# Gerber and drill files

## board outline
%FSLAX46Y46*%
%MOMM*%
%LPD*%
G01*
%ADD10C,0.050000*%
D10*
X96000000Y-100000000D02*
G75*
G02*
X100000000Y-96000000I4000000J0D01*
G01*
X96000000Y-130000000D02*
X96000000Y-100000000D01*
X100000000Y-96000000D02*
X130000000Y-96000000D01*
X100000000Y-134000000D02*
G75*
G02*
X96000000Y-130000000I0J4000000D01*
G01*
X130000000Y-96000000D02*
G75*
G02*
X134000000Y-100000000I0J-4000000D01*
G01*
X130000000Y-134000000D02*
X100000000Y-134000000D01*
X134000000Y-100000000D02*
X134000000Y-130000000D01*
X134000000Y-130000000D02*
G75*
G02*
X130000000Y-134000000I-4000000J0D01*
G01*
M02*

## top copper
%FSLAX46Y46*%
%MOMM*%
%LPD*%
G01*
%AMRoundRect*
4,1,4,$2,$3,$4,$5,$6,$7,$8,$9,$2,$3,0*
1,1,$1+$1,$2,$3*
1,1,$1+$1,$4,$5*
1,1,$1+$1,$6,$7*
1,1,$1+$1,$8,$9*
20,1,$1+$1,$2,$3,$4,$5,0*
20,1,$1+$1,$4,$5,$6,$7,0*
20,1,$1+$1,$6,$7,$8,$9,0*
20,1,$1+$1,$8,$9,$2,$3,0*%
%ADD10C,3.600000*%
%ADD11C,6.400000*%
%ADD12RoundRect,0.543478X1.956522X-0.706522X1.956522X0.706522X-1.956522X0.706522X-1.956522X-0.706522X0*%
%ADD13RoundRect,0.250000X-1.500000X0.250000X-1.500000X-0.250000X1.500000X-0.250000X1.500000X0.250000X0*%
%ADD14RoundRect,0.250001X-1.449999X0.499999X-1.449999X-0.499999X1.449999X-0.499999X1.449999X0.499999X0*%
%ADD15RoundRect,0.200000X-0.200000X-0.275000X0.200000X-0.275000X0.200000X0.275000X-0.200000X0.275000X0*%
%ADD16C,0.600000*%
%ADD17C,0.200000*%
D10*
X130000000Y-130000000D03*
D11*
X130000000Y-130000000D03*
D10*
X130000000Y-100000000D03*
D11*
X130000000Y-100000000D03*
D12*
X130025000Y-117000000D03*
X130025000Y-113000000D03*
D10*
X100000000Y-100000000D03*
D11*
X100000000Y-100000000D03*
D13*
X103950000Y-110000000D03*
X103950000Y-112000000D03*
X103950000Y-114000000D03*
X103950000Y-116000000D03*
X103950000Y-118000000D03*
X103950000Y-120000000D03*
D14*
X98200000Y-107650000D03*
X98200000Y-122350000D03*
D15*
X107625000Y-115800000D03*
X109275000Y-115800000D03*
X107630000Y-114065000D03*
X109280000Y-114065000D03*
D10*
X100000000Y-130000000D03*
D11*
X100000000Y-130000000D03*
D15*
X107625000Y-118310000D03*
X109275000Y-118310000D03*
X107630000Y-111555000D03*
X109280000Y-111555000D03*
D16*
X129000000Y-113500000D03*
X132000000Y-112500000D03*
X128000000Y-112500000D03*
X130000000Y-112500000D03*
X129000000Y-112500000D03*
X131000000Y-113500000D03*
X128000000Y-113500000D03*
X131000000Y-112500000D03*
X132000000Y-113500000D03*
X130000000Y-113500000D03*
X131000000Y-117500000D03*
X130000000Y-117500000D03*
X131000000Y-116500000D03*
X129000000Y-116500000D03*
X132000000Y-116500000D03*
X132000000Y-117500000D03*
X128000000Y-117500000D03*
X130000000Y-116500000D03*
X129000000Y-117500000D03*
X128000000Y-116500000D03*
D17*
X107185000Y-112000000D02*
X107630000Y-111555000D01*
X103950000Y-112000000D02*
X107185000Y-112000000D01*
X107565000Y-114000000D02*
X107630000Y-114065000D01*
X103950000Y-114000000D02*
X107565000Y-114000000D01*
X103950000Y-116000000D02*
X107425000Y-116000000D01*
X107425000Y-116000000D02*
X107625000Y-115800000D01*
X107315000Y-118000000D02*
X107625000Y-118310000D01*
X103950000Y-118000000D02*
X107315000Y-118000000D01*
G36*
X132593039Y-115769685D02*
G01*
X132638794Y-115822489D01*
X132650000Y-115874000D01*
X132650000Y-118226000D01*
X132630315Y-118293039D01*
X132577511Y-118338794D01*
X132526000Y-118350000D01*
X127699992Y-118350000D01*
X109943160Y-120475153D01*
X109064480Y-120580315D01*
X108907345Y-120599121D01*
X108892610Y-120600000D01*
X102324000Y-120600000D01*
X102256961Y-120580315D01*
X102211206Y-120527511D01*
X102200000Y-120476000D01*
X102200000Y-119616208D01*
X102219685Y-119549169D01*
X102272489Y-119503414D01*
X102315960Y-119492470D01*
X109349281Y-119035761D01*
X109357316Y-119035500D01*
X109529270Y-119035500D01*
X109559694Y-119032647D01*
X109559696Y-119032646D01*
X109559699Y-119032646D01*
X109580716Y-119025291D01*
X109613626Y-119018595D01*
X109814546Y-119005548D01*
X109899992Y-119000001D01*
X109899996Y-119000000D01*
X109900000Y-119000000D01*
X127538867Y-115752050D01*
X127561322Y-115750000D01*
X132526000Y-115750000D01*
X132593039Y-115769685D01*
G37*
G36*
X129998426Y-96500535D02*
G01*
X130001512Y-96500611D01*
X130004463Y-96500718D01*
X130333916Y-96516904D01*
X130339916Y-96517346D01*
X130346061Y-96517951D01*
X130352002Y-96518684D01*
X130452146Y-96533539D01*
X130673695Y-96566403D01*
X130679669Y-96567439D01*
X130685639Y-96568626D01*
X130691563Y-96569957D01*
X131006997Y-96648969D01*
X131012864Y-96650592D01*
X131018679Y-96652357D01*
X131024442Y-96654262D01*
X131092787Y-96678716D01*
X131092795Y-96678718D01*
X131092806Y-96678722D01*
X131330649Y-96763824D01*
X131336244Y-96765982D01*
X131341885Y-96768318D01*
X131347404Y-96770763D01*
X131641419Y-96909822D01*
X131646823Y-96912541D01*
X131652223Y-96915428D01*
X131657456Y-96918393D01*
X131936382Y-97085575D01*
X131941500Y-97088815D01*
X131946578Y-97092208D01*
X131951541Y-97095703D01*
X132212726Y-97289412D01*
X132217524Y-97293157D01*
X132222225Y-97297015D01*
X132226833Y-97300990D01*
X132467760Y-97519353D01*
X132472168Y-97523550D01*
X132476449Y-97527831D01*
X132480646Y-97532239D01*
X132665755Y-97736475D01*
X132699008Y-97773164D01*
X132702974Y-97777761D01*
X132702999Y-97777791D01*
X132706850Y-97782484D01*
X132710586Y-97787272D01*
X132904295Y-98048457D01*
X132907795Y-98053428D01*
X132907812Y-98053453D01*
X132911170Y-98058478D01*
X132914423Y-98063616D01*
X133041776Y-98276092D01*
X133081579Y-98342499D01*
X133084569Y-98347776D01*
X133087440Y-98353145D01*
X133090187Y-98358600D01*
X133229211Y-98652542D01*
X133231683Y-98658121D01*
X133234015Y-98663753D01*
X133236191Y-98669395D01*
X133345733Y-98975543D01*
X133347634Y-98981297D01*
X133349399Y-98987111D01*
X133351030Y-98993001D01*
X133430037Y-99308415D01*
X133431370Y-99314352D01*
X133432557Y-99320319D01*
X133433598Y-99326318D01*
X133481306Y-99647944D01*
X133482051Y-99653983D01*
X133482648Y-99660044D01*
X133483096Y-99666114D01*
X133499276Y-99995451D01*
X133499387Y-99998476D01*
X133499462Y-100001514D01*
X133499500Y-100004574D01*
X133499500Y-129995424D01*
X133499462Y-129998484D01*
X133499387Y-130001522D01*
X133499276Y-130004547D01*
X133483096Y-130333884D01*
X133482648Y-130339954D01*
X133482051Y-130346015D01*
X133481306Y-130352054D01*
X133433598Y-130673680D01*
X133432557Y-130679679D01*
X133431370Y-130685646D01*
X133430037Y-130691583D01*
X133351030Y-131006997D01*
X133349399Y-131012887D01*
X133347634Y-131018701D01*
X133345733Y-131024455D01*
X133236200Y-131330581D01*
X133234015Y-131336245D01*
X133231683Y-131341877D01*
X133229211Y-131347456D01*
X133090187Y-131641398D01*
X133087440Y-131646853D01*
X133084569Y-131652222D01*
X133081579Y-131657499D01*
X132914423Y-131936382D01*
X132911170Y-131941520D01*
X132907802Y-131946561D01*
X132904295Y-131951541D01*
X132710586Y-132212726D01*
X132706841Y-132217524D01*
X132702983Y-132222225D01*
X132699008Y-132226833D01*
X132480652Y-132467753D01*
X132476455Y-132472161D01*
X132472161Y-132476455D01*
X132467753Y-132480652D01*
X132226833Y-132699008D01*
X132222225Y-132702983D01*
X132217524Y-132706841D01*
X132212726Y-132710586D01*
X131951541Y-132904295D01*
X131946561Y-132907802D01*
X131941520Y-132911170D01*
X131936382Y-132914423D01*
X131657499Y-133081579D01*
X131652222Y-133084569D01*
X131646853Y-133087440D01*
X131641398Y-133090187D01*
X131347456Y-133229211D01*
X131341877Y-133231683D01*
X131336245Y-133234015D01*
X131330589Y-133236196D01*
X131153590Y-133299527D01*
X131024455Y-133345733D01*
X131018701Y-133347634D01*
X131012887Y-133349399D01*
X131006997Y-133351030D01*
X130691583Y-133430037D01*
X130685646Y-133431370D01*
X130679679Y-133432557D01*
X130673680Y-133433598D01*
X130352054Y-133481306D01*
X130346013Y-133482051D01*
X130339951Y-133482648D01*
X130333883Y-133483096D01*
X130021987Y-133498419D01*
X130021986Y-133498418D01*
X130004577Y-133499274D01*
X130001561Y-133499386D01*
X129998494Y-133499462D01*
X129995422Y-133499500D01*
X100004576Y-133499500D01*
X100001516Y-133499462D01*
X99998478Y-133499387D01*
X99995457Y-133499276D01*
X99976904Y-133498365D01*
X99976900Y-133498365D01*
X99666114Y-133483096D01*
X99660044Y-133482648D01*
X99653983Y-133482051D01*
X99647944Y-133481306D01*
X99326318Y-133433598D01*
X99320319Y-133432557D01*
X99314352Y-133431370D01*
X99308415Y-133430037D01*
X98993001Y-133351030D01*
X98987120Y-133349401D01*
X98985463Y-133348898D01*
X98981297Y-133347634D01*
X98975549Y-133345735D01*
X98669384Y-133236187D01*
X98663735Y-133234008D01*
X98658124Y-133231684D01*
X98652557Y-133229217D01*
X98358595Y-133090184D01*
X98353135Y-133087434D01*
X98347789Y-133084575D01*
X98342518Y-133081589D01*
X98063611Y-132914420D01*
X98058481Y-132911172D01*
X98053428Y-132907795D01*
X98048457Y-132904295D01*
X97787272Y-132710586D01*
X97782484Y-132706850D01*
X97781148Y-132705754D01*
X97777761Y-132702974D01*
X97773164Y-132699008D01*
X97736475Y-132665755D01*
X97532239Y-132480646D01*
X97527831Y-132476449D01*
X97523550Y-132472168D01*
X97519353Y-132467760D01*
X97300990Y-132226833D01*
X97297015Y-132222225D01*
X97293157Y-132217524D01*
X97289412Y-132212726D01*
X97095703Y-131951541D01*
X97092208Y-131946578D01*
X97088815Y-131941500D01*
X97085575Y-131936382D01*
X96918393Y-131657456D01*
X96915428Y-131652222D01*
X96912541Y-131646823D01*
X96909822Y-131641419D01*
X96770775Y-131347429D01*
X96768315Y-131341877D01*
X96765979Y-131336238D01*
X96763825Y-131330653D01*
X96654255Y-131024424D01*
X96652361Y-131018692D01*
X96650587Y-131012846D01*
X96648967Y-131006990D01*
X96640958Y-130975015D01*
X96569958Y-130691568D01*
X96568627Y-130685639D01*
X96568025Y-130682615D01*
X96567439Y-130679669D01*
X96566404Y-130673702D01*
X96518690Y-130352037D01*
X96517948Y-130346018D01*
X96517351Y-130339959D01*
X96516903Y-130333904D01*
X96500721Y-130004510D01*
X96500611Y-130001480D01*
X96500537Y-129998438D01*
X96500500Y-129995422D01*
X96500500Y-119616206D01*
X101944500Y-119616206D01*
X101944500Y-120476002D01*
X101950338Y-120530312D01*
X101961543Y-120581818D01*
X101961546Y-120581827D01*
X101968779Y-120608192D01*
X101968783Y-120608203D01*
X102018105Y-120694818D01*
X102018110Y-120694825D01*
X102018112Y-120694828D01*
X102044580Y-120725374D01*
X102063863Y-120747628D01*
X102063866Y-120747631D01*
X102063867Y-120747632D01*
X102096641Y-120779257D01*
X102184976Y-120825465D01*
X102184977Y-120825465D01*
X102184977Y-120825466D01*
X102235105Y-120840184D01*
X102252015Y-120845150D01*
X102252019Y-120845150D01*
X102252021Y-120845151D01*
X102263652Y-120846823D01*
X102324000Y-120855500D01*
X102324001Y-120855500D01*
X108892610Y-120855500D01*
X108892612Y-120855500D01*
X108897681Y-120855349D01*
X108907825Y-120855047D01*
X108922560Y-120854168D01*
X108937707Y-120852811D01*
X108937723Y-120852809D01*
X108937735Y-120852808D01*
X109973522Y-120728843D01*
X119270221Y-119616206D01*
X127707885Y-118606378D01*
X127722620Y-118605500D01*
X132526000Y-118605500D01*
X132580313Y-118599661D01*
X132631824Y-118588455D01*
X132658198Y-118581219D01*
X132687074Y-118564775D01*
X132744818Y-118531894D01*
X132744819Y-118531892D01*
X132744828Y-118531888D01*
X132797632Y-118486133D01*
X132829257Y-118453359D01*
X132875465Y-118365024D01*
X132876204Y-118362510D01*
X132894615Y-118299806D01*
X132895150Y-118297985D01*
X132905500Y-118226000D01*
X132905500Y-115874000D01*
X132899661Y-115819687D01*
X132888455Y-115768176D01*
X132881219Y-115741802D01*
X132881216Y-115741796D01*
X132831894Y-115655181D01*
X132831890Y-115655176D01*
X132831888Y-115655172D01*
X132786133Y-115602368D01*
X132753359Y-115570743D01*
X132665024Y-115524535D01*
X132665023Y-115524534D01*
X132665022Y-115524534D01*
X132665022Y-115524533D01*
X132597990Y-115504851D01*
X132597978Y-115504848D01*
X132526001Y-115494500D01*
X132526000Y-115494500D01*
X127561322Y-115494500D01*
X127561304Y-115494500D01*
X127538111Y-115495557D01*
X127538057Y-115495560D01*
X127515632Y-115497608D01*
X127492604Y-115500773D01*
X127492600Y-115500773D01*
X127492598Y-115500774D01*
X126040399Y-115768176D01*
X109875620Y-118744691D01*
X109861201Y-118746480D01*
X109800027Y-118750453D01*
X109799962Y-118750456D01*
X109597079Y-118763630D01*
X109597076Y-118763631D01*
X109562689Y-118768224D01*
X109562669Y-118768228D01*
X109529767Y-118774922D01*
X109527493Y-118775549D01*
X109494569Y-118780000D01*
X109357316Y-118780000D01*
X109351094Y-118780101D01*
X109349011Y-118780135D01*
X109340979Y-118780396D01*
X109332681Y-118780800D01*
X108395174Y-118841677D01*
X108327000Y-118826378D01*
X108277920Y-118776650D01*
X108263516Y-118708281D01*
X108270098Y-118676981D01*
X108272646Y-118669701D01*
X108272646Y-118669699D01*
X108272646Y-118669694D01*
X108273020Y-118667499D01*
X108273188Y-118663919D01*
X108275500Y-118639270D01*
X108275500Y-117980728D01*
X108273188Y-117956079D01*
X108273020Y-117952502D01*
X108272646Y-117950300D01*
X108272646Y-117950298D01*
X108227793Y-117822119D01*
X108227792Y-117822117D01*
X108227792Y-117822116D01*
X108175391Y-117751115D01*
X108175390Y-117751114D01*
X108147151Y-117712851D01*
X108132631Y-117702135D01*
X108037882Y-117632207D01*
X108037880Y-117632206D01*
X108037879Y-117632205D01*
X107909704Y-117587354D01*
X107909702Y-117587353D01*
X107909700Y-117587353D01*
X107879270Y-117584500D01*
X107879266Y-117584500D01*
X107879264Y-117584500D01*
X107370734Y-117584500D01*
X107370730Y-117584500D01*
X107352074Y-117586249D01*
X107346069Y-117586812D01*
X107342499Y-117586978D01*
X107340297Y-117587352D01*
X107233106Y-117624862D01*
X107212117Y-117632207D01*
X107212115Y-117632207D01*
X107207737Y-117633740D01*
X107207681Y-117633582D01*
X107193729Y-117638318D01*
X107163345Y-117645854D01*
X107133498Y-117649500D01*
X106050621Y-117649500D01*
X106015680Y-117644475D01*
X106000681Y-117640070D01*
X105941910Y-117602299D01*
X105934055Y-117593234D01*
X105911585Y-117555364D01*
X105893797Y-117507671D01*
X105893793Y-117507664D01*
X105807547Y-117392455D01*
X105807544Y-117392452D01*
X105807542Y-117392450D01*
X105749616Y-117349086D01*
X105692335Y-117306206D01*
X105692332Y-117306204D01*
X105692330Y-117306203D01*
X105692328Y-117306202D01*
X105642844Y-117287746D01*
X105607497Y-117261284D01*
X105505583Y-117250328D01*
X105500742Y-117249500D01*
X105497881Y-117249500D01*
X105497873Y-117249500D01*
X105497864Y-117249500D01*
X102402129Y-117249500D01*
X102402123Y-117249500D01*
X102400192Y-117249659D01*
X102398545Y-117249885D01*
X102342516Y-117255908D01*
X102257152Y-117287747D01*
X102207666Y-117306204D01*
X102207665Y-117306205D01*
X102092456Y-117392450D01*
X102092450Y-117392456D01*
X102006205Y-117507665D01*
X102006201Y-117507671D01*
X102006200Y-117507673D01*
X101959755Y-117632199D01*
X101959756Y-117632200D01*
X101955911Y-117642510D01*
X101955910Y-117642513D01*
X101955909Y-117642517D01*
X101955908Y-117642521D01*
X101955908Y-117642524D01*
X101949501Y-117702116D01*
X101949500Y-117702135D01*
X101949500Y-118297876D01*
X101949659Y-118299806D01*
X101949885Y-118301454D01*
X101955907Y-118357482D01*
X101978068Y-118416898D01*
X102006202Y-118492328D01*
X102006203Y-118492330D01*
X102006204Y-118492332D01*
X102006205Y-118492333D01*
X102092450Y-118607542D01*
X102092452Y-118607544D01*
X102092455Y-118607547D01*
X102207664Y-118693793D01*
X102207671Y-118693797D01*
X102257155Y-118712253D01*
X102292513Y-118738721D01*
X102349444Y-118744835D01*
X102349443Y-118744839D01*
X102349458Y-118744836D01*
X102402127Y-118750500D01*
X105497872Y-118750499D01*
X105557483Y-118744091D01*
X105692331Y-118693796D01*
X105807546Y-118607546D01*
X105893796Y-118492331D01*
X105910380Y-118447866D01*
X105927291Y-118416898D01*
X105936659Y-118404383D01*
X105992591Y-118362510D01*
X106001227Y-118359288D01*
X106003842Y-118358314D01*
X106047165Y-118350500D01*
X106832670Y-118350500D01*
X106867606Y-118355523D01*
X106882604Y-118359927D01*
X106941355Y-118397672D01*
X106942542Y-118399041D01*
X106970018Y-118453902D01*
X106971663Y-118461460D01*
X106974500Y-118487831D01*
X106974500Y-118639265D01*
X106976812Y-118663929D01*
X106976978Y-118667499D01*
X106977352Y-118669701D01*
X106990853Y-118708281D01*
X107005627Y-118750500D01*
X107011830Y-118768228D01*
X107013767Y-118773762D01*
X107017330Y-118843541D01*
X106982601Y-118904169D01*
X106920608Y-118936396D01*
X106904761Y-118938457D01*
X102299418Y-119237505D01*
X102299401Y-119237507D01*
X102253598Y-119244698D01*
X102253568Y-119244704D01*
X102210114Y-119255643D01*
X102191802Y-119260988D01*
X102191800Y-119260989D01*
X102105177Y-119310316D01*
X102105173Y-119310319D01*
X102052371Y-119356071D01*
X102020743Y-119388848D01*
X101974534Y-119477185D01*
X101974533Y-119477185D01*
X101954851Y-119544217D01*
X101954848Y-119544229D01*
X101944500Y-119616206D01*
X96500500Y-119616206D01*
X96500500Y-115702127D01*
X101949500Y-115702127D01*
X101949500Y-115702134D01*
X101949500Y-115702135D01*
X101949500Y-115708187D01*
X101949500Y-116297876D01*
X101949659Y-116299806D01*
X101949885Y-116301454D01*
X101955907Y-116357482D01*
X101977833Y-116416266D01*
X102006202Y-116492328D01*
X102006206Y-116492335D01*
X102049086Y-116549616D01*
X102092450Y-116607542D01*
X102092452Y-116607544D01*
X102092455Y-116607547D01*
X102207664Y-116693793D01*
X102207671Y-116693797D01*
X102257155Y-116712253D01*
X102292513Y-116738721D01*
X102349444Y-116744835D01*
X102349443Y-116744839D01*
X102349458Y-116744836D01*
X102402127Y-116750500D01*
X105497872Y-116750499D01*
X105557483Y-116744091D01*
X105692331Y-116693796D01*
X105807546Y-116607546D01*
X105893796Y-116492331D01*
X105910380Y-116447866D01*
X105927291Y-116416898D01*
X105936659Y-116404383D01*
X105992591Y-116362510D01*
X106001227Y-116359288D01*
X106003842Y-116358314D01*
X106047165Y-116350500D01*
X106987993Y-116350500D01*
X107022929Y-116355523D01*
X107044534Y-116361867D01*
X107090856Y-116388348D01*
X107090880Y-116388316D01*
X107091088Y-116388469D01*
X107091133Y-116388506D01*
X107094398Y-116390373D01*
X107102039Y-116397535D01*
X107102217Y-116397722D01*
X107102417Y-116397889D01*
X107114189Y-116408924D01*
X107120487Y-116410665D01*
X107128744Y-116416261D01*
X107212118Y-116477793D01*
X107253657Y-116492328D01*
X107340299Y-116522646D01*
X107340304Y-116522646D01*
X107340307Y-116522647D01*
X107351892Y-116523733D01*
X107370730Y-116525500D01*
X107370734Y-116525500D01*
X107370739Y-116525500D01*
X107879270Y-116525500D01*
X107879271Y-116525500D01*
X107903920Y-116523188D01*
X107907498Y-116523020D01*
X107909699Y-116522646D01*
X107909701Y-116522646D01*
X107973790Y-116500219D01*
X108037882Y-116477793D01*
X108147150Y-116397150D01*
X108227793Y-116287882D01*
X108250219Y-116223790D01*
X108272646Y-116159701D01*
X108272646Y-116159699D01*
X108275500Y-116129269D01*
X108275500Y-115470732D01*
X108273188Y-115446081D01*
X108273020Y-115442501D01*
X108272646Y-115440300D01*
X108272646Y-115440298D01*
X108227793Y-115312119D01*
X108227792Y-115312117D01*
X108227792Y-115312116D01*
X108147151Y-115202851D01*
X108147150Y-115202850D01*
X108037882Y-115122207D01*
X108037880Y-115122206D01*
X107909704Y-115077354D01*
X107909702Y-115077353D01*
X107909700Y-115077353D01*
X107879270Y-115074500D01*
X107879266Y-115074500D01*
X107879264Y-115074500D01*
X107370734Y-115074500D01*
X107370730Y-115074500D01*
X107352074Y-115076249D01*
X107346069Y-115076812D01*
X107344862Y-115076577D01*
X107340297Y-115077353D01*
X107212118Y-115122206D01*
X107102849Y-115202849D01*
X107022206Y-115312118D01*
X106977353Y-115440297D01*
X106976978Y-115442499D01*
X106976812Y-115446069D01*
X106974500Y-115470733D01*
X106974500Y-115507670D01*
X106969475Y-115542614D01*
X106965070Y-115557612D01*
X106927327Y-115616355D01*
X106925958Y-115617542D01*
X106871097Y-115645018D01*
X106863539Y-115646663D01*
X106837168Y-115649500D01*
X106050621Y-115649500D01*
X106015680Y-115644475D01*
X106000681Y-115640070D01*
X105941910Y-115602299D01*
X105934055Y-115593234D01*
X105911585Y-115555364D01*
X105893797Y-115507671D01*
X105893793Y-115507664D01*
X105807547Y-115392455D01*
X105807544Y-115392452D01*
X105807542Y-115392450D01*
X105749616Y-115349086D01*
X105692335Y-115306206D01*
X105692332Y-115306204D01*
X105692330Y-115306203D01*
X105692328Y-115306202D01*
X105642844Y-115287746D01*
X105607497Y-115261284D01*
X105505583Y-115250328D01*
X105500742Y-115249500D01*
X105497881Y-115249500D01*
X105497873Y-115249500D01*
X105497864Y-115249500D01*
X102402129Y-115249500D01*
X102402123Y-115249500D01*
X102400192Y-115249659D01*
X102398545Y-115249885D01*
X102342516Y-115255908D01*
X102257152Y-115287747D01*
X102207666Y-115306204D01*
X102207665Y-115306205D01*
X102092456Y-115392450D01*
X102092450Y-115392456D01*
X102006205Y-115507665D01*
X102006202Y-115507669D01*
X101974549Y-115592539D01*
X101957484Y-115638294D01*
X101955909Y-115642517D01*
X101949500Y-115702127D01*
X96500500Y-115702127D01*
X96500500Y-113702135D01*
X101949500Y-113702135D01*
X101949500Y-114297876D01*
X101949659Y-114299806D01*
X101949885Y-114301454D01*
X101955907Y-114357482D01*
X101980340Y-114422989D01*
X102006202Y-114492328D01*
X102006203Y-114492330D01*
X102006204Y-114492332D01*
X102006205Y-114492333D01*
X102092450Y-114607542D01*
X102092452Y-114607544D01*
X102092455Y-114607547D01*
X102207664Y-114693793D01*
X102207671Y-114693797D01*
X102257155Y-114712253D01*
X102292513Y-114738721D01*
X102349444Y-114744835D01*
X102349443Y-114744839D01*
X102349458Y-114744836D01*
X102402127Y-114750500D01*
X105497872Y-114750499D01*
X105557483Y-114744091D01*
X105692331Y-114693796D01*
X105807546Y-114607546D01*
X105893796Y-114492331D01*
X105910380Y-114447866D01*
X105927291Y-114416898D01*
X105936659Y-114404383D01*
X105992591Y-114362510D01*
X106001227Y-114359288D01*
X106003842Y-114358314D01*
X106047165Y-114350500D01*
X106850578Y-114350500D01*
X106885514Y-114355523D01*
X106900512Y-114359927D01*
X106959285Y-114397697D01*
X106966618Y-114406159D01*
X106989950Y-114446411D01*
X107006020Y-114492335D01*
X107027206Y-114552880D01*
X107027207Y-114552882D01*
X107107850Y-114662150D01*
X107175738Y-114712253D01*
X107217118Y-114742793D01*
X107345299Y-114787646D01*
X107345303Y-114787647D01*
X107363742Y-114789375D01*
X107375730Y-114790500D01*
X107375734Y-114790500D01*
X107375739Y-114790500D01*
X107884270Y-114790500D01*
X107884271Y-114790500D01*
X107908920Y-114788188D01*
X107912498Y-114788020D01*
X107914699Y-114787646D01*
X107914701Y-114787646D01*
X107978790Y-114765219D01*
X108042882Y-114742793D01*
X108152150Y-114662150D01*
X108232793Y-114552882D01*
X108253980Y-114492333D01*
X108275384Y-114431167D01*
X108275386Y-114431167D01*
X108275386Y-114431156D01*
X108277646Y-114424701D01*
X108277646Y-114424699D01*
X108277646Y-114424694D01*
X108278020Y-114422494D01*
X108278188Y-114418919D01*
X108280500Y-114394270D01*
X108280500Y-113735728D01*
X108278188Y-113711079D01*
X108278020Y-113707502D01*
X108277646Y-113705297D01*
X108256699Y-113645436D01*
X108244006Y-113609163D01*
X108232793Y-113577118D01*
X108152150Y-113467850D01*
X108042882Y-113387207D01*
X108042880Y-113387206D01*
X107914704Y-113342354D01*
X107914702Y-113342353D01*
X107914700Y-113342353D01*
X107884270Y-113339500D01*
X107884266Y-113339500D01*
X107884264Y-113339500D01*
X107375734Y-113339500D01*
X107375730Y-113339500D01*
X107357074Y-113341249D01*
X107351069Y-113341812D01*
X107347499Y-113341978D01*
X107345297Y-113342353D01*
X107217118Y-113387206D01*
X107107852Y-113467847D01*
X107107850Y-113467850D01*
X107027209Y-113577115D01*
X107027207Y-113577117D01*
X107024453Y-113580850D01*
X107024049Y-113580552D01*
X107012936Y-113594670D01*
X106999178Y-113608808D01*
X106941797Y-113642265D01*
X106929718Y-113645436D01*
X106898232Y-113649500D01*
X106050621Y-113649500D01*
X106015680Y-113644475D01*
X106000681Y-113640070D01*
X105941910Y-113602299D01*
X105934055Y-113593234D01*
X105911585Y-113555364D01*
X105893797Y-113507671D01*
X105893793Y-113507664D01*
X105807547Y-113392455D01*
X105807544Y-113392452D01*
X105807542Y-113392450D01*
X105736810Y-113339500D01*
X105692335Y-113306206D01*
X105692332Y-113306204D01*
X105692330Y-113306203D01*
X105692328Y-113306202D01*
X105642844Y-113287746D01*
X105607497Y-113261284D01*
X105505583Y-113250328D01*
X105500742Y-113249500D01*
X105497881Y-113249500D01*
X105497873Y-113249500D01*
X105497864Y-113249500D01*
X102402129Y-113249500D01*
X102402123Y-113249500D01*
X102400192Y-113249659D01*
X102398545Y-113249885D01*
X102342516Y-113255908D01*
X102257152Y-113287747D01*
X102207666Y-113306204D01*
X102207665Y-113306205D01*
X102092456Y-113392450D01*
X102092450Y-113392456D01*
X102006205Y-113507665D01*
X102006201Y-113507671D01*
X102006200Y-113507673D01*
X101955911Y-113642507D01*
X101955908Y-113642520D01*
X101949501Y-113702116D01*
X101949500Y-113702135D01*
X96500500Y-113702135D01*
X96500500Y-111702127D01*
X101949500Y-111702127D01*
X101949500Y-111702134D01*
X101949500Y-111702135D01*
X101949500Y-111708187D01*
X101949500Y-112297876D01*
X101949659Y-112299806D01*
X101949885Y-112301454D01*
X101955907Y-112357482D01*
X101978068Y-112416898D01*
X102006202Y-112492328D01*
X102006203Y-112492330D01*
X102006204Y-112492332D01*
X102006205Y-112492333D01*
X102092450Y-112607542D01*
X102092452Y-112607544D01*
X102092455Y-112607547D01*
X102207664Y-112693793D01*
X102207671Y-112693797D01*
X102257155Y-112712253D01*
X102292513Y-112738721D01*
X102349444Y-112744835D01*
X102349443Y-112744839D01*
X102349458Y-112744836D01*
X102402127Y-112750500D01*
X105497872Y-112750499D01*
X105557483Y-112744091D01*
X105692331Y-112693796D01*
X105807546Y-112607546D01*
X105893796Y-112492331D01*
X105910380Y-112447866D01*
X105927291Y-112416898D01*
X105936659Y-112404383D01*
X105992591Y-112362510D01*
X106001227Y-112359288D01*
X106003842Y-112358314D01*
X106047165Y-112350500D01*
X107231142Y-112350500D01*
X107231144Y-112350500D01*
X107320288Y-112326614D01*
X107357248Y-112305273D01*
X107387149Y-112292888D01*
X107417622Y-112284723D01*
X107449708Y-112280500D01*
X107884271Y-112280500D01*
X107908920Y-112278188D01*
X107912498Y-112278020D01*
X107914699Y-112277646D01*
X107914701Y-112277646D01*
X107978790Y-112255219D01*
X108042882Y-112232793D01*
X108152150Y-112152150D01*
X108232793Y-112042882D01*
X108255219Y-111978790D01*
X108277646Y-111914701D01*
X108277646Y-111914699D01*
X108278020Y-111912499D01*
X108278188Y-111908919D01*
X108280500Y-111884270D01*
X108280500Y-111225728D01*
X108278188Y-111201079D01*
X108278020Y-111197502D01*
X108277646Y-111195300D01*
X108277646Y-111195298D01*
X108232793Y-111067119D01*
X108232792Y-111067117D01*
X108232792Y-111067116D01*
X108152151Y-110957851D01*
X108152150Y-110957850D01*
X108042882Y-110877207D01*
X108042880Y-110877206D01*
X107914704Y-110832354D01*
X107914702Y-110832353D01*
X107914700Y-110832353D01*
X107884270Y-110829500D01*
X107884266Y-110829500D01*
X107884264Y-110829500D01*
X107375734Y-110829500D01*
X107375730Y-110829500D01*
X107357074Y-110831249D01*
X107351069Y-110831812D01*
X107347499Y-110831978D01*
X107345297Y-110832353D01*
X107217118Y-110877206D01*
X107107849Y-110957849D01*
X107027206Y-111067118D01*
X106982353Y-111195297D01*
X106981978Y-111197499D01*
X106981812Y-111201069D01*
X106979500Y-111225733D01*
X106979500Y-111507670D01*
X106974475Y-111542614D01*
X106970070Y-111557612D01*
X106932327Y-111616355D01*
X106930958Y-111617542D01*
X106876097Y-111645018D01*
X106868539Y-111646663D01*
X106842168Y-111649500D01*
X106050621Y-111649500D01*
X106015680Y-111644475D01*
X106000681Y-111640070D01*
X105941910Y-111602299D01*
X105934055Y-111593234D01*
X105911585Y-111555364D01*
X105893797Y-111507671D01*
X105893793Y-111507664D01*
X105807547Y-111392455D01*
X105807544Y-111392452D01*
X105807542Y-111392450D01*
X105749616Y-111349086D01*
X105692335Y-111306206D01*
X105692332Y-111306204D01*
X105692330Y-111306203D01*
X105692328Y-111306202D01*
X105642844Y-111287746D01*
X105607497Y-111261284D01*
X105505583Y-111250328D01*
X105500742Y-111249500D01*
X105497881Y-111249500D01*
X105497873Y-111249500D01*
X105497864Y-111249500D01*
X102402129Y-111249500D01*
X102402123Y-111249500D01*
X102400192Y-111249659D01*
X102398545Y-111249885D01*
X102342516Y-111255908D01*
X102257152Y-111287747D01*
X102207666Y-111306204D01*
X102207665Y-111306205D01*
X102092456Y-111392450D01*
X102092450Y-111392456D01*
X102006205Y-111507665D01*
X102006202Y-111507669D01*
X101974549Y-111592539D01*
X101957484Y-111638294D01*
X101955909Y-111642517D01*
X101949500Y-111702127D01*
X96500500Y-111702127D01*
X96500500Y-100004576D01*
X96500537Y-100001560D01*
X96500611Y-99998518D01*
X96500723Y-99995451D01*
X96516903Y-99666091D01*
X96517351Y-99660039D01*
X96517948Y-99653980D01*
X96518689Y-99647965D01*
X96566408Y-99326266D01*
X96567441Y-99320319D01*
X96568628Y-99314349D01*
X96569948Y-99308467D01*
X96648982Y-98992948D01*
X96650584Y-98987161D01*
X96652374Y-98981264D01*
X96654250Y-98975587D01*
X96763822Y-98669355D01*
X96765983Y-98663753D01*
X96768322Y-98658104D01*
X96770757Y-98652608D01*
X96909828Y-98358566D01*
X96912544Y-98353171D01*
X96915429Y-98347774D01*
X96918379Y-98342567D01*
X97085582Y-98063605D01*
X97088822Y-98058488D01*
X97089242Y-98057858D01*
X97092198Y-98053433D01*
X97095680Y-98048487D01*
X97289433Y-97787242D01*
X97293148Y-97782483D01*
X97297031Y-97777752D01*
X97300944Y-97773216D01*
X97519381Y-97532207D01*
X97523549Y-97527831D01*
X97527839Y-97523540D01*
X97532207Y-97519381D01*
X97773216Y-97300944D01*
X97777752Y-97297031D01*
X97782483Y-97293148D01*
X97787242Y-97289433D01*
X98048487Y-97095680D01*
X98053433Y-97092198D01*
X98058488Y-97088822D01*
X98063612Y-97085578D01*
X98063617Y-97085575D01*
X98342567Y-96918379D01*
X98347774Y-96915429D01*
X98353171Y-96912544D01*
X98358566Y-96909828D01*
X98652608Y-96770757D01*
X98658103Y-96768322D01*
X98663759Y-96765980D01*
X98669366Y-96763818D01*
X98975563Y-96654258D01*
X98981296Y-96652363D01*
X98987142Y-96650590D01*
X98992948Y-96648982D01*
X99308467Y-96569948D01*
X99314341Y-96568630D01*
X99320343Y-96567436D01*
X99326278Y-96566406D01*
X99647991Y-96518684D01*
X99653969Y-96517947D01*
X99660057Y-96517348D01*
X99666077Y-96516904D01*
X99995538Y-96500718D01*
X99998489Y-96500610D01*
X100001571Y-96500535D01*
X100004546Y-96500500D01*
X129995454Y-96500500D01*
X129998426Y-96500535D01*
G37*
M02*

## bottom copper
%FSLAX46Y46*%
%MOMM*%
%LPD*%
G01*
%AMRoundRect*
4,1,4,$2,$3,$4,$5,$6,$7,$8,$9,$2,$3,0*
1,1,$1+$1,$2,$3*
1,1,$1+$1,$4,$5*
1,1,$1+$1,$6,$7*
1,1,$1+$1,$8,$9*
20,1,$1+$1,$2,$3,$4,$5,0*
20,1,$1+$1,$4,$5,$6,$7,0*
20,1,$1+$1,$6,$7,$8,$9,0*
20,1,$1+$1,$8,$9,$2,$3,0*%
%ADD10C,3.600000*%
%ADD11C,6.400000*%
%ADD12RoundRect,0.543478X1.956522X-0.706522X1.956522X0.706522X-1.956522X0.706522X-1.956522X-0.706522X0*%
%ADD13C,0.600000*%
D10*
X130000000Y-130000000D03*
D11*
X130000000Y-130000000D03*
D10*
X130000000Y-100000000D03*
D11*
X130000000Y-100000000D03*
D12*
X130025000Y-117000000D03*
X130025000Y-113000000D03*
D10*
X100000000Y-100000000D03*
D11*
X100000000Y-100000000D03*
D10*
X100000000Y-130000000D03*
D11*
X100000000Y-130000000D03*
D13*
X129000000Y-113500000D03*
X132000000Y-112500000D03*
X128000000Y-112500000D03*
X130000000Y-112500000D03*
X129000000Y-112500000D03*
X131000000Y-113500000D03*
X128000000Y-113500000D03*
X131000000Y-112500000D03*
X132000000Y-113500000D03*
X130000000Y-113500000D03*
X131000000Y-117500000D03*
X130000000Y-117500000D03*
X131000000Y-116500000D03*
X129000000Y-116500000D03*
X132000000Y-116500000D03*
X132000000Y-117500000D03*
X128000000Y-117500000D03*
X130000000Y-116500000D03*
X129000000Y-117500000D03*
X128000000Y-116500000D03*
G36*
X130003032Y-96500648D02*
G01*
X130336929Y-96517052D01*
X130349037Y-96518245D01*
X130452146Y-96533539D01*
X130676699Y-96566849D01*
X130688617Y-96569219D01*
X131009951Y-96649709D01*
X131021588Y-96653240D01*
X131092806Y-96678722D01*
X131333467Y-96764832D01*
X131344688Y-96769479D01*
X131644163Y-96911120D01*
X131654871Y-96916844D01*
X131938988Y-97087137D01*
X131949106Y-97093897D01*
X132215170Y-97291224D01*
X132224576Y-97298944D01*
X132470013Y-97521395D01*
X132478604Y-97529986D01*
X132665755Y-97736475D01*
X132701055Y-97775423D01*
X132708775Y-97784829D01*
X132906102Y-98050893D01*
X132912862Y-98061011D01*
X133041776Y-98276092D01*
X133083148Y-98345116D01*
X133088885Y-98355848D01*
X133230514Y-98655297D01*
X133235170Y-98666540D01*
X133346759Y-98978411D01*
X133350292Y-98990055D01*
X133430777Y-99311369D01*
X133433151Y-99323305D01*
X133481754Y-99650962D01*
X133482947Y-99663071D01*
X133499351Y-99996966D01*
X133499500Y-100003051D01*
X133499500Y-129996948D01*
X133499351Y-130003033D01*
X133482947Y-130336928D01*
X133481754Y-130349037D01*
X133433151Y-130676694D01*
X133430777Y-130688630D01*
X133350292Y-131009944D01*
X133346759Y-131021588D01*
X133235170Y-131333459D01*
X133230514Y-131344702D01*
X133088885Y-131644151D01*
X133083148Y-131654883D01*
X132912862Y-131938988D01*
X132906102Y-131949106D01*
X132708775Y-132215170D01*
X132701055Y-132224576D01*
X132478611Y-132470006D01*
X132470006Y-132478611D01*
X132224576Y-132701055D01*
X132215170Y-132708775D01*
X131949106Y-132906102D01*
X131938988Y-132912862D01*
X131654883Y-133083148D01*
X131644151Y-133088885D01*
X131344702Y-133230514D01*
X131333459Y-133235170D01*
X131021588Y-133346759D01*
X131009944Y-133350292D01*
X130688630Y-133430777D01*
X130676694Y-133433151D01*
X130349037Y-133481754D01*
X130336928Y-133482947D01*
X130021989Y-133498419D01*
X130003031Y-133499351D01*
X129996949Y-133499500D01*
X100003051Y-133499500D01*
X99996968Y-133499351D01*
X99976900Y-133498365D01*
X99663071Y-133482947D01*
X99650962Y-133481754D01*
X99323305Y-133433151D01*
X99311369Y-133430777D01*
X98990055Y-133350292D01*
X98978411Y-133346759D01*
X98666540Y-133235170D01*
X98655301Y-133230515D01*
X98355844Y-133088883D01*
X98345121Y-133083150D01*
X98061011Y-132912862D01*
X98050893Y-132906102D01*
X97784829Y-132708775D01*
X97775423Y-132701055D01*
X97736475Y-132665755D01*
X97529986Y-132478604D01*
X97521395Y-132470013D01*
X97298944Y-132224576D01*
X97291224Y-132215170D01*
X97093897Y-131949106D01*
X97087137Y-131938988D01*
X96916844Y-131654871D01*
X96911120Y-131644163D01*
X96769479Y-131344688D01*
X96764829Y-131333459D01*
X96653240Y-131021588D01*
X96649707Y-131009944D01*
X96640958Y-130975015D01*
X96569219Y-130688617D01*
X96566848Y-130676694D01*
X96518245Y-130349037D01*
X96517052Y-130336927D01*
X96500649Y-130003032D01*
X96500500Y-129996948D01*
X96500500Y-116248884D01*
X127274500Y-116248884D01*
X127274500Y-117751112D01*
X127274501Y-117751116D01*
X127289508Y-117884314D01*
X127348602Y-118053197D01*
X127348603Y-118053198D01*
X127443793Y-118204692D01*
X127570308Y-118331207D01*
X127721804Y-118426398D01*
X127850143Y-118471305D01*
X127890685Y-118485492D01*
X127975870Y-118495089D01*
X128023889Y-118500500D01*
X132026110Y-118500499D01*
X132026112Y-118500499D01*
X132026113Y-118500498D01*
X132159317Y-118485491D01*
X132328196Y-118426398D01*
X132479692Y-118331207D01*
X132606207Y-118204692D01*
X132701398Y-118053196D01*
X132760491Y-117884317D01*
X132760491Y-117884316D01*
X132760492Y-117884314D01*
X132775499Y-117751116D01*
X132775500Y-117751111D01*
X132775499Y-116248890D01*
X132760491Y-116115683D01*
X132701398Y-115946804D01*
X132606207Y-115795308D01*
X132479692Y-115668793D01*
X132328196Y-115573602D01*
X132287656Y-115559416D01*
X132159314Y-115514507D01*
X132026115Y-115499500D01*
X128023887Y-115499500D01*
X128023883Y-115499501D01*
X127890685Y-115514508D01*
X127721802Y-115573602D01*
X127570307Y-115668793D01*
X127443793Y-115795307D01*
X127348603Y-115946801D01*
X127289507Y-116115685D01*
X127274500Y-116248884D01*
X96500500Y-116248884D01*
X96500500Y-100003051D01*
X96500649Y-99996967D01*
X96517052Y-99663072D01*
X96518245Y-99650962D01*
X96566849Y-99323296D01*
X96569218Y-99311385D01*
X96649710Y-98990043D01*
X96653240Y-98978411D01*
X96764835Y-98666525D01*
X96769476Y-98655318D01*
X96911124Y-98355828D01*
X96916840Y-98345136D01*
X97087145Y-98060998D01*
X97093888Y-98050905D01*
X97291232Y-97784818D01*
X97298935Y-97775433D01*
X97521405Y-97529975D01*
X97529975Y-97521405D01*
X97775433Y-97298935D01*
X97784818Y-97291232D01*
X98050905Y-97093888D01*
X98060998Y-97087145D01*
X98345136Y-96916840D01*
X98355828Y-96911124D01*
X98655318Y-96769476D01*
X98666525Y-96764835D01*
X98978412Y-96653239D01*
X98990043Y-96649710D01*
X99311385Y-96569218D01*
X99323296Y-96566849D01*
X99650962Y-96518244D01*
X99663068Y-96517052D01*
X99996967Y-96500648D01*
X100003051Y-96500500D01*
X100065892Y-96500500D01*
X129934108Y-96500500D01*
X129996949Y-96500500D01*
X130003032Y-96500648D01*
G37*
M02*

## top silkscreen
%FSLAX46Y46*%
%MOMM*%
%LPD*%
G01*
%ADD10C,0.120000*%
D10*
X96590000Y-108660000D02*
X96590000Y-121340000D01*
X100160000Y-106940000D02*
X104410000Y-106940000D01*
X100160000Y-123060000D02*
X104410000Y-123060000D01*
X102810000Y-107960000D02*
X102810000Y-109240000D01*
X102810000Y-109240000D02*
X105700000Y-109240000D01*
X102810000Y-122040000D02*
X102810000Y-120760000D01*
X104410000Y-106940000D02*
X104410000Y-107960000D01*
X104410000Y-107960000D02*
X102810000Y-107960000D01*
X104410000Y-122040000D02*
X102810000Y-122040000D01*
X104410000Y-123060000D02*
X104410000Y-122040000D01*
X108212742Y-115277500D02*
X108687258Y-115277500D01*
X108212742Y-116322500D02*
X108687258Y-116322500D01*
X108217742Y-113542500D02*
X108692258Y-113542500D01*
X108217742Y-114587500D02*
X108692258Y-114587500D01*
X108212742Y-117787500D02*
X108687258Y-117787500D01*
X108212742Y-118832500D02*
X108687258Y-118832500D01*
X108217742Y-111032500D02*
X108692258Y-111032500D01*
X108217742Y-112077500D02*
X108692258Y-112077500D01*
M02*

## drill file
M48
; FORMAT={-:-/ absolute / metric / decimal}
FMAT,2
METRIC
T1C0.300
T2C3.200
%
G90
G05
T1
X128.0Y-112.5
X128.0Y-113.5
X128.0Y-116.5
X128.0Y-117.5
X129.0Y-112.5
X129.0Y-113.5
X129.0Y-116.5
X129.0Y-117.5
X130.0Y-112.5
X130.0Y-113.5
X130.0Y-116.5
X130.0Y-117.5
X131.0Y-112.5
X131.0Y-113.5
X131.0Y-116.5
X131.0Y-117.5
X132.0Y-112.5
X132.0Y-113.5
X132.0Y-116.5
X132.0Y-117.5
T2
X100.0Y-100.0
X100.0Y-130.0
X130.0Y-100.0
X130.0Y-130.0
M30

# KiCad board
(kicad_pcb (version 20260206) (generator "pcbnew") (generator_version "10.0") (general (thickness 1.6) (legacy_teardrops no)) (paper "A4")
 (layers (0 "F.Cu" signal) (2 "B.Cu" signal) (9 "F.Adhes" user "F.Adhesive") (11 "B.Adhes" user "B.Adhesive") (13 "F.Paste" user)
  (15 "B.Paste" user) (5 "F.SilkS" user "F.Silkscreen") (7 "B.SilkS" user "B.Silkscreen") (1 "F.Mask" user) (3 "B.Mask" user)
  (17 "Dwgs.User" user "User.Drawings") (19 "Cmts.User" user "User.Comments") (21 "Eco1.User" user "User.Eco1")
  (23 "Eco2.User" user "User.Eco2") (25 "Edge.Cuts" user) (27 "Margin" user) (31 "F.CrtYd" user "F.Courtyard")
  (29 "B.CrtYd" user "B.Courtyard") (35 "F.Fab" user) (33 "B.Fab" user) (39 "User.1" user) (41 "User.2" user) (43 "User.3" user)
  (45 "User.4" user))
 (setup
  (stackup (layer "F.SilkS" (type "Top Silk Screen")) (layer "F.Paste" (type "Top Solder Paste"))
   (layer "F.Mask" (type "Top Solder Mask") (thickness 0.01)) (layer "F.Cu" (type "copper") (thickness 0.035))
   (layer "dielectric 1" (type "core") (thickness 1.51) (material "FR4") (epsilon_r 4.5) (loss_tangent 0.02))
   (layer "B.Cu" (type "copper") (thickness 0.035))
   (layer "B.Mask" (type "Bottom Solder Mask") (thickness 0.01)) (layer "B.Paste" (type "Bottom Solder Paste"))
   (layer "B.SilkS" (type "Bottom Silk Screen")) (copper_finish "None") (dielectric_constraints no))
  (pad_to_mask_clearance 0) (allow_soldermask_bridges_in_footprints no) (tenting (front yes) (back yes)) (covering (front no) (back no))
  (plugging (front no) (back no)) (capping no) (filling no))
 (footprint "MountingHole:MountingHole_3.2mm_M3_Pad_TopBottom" (layer "F.Cu") (at 130 130)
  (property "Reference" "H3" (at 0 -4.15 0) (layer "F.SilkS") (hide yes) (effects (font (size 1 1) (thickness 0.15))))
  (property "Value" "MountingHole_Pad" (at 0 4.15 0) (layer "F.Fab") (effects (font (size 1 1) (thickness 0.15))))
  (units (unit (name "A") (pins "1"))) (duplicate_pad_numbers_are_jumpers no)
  (pad "1" thru_hole circle (at 0 0) (size 3.6 3.6) (drill 3.2) (layers "*.Cu" "*.Mask") (remove_unused_layers no) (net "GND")
   (zone_connect 2))
  (pad "1" connect circle (at 0 0) (size 6.4 6.4) (layers "F.Cu" "F.Mask") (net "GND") (zone_connect 2))
  (pad "1" connect circle (at 0 0) (size 6.4 6.4) (layers "B.Cu" "B.Mask") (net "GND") (zone_connect 2)))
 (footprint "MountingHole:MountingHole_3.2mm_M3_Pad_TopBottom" (layer "F.Cu") (at 130 100)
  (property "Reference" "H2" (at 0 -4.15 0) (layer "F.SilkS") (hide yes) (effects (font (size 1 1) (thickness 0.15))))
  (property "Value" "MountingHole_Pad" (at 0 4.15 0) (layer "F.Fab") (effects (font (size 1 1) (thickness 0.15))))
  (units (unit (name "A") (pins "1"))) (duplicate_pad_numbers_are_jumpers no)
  (pad "1" thru_hole circle (at 0 0) (size 3.6 3.6) (drill 3.2) (layers "*.Cu" "*.Mask") (remove_unused_layers no) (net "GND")
   (zone_connect 2))
  (pad "1" connect circle (at 0 0) (size 6.4 6.4) (layers "F.Cu" "F.Mask") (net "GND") (zone_connect 2))
  (pad "1" connect circle (at 0 0) (size 6.4 6.4) (layers "B.Cu" "B.Mask") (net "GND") (zone_connect 2)))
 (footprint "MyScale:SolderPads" (layer "F.Cu") (at 130.025 115 90)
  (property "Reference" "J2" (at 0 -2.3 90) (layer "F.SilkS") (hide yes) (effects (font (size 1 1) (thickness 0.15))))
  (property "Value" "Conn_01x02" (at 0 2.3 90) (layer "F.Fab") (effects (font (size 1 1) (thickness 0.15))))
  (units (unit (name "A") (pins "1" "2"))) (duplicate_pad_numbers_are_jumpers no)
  (pad "1" smd roundrect (at -2 0 90) (size 2.5 5) (layers "F.Cu" "F.Mask") (roundrect_rratio 0.217391) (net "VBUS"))
  (pad "1" smd roundrect (at -2 0 90) (size 2.5 5) (layers "B.Cu") (roundrect_rratio 0.217391) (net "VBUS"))
  (pad "2" smd roundrect (at 2 0 90) (size 2.5 5) (layers "F.Cu" "F.Mask") (roundrect_rratio 0.217391) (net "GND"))
  (pad "2" smd roundrect (at 2 0 90) (size 2.5 5) (layers "B.Cu") (roundrect_rratio 0.217391) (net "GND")))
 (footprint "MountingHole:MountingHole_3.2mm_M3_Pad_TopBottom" (layer "F.Cu") (at 100 100)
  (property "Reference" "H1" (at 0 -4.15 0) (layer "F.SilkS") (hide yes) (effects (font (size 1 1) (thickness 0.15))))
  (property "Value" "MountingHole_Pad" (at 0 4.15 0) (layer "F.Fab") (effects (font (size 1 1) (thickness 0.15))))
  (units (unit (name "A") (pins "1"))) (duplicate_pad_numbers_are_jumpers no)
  (pad "1" thru_hole circle (at 0 0) (size 3.6 3.6) (drill 3.2) (layers "*.Cu" "*.Mask") (remove_unused_layers no) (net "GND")
   (zone_connect 2))
  (pad "1" connect circle (at 0 0) (size 6.4 6.4) (layers "F.Cu" "F.Mask") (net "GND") (zone_connect 2))
  (pad "1" connect circle (at 0 0) (size 6.4 6.4) (layers "B.Cu" "B.Mask") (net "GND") (zone_connect 2)))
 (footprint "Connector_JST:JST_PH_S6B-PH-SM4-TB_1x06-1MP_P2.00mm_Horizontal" (layer "F.Cu") (at 101.1 115 -90)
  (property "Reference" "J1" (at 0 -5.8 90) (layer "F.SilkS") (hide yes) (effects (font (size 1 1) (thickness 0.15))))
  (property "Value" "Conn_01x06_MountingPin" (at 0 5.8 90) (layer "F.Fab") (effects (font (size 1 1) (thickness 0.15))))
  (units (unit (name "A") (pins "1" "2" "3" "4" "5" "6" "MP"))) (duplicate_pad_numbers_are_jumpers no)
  (fp_line (start -6.34 4.51) (end 6.34 4.51) (stroke (width 0.12) (type solid)) (layer "F.SilkS"))
  (fp_line (start -8.06 0.94) (end -8.06 -3.31) (stroke (width 0.12) (type solid)) (layer "F.SilkS"))
  (fp_line (start 8.06 0.94) (end 8.06 -3.31) (stroke (width 0.12) (type solid)) (layer "F.SilkS"))
  (fp_line (start -7.04 -1.71) (end -5.76 -1.71) (stroke (width 0.12) (type solid)) (layer "F.SilkS"))
  (fp_line (start -5.76 -1.71) (end -5.76 -4.6) (stroke (width 0.12) (type solid)) (layer "F.SilkS"))
  (fp_line (start 7.04 -1.71) (end 5.76 -1.71) (stroke (width 0.12) (type solid)) (layer "F.SilkS"))
  (fp_line (start -8.06 -3.31) (end -7.04 -3.31) (stroke (width 0.12) (type solid)) (layer "F.SilkS"))
  (fp_line (start -7.04 -3.31) (end -7.04 -1.71) (stroke (width 0.12) (type solid)) (layer "F.SilkS"))
  (fp_line (start 7.04 -3.31) (end 7.04 -1.71) (stroke (width 0.12) (type solid)) (layer "F.SilkS"))
  (fp_line (start 8.06 -3.31) (end 7.04 -3.31) (stroke (width 0.12) (type solid)) (layer "F.SilkS"))
  (pad "1" smd roundrect (at -5 -2.85 270) (size 1 3.5) (layers "F.Cu" "F.Mask" "F.Paste") (roundrect_rratio 0.25) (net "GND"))
  (pad "2" smd roundrect (at -3 -2.85 270) (size 1 3.5) (layers "F.Cu" "F.Mask" "F.Paste") (roundrect_rratio 0.25) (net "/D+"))
  (pad "3" smd roundrect (at -1 -2.85 270) (size 1 3.5) (layers "F.Cu" "F.Mask" "F.Paste") (roundrect_rratio 0.25) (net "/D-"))
  (pad "4" smd roundrect (at 1 -2.85 270) (size 1 3.5) (layers "F.Cu" "F.Mask" "F.Paste") (roundrect_rratio 0.25) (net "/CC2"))
  (pad "5" smd roundrect (at 3 -2.85 270) (size 1 3.5) (layers "F.Cu" "F.Mask" "F.Paste") (roundrect_rratio 0.25) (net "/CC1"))
  (pad "6" smd roundrect (at 5 -2.85 270) (size 1 3.5) (layers "F.Cu" "F.Mask" "F.Paste") (roundrect_rratio 0.25) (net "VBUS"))
  (pad "MP" smd roundrect (at -7.35 2.9 270) (size 1.5 3.4) (layers "F.Cu" "F.Mask" "F.Paste") (roundrect_rratio 0.166667) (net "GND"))
  (pad "MP" smd roundrect (at 7.35 2.9 270) (size 1.5 3.4) (layers "F.Cu" "F.Mask" "F.Paste") (roundrect_rratio 0.166667) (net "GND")))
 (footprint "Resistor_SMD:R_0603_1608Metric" (layer "F.Cu") (at 108.45 115.8)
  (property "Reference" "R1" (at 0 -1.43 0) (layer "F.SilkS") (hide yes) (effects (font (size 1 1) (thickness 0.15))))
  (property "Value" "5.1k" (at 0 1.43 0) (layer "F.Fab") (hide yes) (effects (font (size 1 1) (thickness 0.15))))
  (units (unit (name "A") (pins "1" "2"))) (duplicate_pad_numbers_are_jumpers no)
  (fp_line (start -0.237258 -0.5225) (end 0.237258 -0.5225) (stroke (width 0.12) (type solid)) (layer "F.SilkS"))
  (fp_line (start -0.237258 0.5225) (end 0.237258 0.5225) (stroke (width 0.12) (type solid)) (layer "F.SilkS"))
  (pad "1" smd roundrect (at -0.825 0) (size 0.8 0.95) (layers "F.Cu" "F.Mask" "F.Paste") (roundrect_rratio 0.25) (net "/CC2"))
  (pad "2" smd roundrect (at 0.825 0) (size 0.8 0.95) (layers "F.Cu" "F.Mask" "F.Paste") (roundrect_rratio 0.25) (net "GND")))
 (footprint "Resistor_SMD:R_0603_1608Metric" (layer "F.Cu") (at 108.455 114.065)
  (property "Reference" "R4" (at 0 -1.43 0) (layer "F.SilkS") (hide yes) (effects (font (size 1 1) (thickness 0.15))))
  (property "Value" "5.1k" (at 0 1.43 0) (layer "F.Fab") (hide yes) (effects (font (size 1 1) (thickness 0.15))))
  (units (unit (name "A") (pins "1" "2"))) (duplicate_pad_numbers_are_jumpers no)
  (fp_line (start -0.237258 -0.5225) (end 0.237258 -0.5225) (stroke (width 0.12) (type solid)) (layer "F.SilkS"))
  (fp_line (start -0.237258 0.5225) (end 0.237258 0.5225) (stroke (width 0.12) (type solid)) (layer "F.SilkS"))
  (pad "1" smd roundrect (at -0.825 0) (size 0.8 0.95) (layers "F.Cu" "F.Mask" "F.Paste") (roundrect_rratio 0.25) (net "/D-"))
  (pad "2" smd roundrect (at 0.825 0) (size 0.8 0.95) (layers "F.Cu" "F.Mask" "F.Paste") (roundrect_rratio 0.25) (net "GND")))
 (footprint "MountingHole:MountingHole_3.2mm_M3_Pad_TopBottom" (layer "F.Cu") (at 100 130)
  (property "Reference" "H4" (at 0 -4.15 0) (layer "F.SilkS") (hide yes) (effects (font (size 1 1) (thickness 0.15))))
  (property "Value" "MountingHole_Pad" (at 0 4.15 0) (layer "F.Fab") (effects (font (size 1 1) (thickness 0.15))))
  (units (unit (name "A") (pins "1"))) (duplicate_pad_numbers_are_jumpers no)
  (pad "1" thru_hole circle (at 0 0) (size 3.6 3.6) (drill 3.2) (layers "*.Cu" "*.Mask") (remove_unused_layers no) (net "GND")
   (zone_connect 2))
  (pad "1" connect circle (at 0 0) (size 6.4 6.4) (layers "F.Cu" "F.Mask") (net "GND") (zone_connect 2))
  (pad "1" connect circle (at 0 0) (size 6.4 6.4) (layers "B.Cu" "B.Mask") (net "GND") (zone_connect 2)))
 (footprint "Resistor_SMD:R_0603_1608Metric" (layer "F.Cu") (at 108.45 118.31)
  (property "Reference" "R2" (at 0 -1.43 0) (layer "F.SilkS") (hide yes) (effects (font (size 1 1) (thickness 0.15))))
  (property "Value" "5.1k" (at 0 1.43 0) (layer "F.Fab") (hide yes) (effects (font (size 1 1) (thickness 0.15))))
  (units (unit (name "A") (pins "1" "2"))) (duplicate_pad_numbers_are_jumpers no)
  (fp_line (start -0.237258 -0.5225) (end 0.237258 -0.5225) (stroke (width 0.12) (type solid)) (layer "F.SilkS"))
  (fp_line (start -0.237258 0.5225) (end 0.237258 0.5225) (stroke (width 0.12) (type solid)) (layer "F.SilkS"))
  (pad "1" smd roundrect (at -0.825 0) (size 0.8 0.95) (layers "F.Cu" "F.Mask" "F.Paste") (roundrect_rratio 0.25) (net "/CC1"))
  (pad "2" smd roundrect (at 0.825 0) (size 0.8 0.95) (layers "F.Cu" "F.Mask" "F.Paste") (roundrect_rratio 0.25) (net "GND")))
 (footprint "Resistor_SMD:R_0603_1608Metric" (layer "F.Cu") (at 108.455 111.555)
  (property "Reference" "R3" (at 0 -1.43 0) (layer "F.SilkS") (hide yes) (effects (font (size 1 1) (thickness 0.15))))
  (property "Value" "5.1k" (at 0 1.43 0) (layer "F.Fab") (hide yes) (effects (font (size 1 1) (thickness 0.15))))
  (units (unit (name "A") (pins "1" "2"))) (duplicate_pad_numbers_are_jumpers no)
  (fp_line (start -0.237258 -0.5225) (end 0.237258 -0.5225) (stroke (width 0.12) (type solid)) (layer "F.SilkS"))
  (fp_line (start -0.237258 0.5225) (end 0.237258 0.5225) (stroke (width 0.12) (type solid)) (layer "F.SilkS"))
  (pad "1" smd roundrect (at -0.825 0) (size 0.8 0.95) (layers "F.Cu" "F.Mask" "F.Paste") (roundrect_rratio 0.25) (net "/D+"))
  (pad "2" smd roundrect (at 0.825 0) (size 0.8 0.95) (layers "F.Cu" "F.Mask" "F.Paste") (roundrect_rratio 0.25) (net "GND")))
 (gr_arc (start 96 100) (mid 97.171573 97.171573) (end 100 96) (stroke (width 0.05) (type default)) (layer "Edge.Cuts"))
 (gr_line (start 96 130) (end 96 100) (stroke (width 0.05) (type default)) (layer "Edge.Cuts"))
 (gr_line (start 100 96) (end 130 96) (stroke (width 0.05) (type default)) (layer "Edge.Cuts"))
 (gr_arc (start 100 134) (mid 97.171573 132.828427) (end 96 130) (stroke (width 0.05) (type default)) (layer "Edge.Cuts"))
 (gr_arc (start 130 96) (mid 132.828427 97.171573) (end 134 100) (stroke (width 0.05) (type default)) (layer "Edge.Cuts"))
 (gr_line (start 130 134) (end 100 134) (stroke (width 0.05) (type default)) (layer "Edge.Cuts"))
 (gr_line (start 134 100) (end 134 130) (stroke (width 0.05) (type default)) (layer "Edge.Cuts"))
 (gr_arc (start 134 130) (mid 132.828427 132.828427) (end 130 134) (stroke (width 0.05) (type default)) (layer "Edge.Cuts"))
 (via (at 129 113.5) (size 0.6) (drill 0.3) (layers "F.Cu" "B.Cu") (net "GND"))
 (via (at 132 112.5) (size 0.6) (drill 0.3) (layers "F.Cu" "B.Cu") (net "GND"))
 (via (at 128 112.5) (size 0.6) (drill 0.3) (layers "F.Cu" "B.Cu") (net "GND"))
 (via (at 130 112.5) (size 0.6) (drill 0.3) (layers "F.Cu" "B.Cu") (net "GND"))
 (via (at 129 112.5) (size 0.6) (drill 0.3) (layers "F.Cu" "B.Cu") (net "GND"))
 (via (at 131 113.5) (size 0.6) (drill 0.3) (layers "F.Cu" "B.Cu") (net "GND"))
 (via (at 128 113.5) (size 0.6) (drill 0.3) (layers "F.Cu" "B.Cu") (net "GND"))
 (via (at 131 112.5) (size 0.6) (drill 0.3) (layers "F.Cu" "B.Cu") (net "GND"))
 (via (at 132 113.5) (size 0.6) (drill 0.3) (layers "F.Cu" "B.Cu") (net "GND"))
 (via (at 130 113.5) (size 0.6) (drill 0.3) (layers "F.Cu" "B.Cu") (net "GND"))
 (via (at 131 117.5) (size 0.6) (drill 0.3) (layers "F.Cu" "B.Cu") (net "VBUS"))
 (via (at 130 117.5) (size 0.6) (drill 0.3) (layers "F.Cu" "B.Cu") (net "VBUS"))
 (via (at 131 116.5) (size 0.6) (drill 0.3) (layers "F.Cu" "B.Cu") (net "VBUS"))
 (via (at 129 116.5) (size 0.6) (drill 0.3) (layers "F.Cu" "B.Cu") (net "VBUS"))
 (via (at 132 116.5) (size 0.6) (drill 0.3) (layers "F.Cu" "B.Cu") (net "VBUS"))
 (via (at 132 117.5) (size 0.6) (drill 0.3) (layers "F.Cu" "B.Cu") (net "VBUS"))
 (via (at 128 117.5) (size 0.6) (drill 0.3) (layers "F.Cu" "B.Cu") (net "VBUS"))
 (via (at 130 116.5) (size 0.6) (drill 0.3) (layers "F.Cu" "B.Cu") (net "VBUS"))
 (via (at 129 117.5) (size 0.6) (drill 0.3) (layers "F.Cu" "B.Cu") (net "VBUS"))
 (via (at 128 116.5) (size 0.6) (drill 0.3) (layers "F.Cu" "B.Cu") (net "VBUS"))
 (segment (start 107.185 112) (end 107.63 111.555) (width 0.2) (layer "F.Cu") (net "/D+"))
 (segment (start 103.95 112) (end 107.185 112) (width 0.2) (layer "F.Cu") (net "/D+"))
 (segment (start 107.565 114) (end 107.63 114.065) (width 0.2) (layer "F.Cu") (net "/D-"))
 (segment (start 103.95 114) (end 107.565 114) (width 0.2) (layer "F.Cu") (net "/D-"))
 (segment (start 103.95 116) (end 107.425 116) (width 0.2) (layer "F.Cu") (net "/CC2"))
 (segment (start 107.425 116) (end 107.625 115.8) (width 0.2) (layer "F.Cu") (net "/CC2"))
 (segment (start 107.315 118) (end 107.625 118.31) (width 0.2) (layer "F.Cu") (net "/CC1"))
 (segment (start 103.95 118) (end 107.315 118) (width 0.2) (layer "F.Cu") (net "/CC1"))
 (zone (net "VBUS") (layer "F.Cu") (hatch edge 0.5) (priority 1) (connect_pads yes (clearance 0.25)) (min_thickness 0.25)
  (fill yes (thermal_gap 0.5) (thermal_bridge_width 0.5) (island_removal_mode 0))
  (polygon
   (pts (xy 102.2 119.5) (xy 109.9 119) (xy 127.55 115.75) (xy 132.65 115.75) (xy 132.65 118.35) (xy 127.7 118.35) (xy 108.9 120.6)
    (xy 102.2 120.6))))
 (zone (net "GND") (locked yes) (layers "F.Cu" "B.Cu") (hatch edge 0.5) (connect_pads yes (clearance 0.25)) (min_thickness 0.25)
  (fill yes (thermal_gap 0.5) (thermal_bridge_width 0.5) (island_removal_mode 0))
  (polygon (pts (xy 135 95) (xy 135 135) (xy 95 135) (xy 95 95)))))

